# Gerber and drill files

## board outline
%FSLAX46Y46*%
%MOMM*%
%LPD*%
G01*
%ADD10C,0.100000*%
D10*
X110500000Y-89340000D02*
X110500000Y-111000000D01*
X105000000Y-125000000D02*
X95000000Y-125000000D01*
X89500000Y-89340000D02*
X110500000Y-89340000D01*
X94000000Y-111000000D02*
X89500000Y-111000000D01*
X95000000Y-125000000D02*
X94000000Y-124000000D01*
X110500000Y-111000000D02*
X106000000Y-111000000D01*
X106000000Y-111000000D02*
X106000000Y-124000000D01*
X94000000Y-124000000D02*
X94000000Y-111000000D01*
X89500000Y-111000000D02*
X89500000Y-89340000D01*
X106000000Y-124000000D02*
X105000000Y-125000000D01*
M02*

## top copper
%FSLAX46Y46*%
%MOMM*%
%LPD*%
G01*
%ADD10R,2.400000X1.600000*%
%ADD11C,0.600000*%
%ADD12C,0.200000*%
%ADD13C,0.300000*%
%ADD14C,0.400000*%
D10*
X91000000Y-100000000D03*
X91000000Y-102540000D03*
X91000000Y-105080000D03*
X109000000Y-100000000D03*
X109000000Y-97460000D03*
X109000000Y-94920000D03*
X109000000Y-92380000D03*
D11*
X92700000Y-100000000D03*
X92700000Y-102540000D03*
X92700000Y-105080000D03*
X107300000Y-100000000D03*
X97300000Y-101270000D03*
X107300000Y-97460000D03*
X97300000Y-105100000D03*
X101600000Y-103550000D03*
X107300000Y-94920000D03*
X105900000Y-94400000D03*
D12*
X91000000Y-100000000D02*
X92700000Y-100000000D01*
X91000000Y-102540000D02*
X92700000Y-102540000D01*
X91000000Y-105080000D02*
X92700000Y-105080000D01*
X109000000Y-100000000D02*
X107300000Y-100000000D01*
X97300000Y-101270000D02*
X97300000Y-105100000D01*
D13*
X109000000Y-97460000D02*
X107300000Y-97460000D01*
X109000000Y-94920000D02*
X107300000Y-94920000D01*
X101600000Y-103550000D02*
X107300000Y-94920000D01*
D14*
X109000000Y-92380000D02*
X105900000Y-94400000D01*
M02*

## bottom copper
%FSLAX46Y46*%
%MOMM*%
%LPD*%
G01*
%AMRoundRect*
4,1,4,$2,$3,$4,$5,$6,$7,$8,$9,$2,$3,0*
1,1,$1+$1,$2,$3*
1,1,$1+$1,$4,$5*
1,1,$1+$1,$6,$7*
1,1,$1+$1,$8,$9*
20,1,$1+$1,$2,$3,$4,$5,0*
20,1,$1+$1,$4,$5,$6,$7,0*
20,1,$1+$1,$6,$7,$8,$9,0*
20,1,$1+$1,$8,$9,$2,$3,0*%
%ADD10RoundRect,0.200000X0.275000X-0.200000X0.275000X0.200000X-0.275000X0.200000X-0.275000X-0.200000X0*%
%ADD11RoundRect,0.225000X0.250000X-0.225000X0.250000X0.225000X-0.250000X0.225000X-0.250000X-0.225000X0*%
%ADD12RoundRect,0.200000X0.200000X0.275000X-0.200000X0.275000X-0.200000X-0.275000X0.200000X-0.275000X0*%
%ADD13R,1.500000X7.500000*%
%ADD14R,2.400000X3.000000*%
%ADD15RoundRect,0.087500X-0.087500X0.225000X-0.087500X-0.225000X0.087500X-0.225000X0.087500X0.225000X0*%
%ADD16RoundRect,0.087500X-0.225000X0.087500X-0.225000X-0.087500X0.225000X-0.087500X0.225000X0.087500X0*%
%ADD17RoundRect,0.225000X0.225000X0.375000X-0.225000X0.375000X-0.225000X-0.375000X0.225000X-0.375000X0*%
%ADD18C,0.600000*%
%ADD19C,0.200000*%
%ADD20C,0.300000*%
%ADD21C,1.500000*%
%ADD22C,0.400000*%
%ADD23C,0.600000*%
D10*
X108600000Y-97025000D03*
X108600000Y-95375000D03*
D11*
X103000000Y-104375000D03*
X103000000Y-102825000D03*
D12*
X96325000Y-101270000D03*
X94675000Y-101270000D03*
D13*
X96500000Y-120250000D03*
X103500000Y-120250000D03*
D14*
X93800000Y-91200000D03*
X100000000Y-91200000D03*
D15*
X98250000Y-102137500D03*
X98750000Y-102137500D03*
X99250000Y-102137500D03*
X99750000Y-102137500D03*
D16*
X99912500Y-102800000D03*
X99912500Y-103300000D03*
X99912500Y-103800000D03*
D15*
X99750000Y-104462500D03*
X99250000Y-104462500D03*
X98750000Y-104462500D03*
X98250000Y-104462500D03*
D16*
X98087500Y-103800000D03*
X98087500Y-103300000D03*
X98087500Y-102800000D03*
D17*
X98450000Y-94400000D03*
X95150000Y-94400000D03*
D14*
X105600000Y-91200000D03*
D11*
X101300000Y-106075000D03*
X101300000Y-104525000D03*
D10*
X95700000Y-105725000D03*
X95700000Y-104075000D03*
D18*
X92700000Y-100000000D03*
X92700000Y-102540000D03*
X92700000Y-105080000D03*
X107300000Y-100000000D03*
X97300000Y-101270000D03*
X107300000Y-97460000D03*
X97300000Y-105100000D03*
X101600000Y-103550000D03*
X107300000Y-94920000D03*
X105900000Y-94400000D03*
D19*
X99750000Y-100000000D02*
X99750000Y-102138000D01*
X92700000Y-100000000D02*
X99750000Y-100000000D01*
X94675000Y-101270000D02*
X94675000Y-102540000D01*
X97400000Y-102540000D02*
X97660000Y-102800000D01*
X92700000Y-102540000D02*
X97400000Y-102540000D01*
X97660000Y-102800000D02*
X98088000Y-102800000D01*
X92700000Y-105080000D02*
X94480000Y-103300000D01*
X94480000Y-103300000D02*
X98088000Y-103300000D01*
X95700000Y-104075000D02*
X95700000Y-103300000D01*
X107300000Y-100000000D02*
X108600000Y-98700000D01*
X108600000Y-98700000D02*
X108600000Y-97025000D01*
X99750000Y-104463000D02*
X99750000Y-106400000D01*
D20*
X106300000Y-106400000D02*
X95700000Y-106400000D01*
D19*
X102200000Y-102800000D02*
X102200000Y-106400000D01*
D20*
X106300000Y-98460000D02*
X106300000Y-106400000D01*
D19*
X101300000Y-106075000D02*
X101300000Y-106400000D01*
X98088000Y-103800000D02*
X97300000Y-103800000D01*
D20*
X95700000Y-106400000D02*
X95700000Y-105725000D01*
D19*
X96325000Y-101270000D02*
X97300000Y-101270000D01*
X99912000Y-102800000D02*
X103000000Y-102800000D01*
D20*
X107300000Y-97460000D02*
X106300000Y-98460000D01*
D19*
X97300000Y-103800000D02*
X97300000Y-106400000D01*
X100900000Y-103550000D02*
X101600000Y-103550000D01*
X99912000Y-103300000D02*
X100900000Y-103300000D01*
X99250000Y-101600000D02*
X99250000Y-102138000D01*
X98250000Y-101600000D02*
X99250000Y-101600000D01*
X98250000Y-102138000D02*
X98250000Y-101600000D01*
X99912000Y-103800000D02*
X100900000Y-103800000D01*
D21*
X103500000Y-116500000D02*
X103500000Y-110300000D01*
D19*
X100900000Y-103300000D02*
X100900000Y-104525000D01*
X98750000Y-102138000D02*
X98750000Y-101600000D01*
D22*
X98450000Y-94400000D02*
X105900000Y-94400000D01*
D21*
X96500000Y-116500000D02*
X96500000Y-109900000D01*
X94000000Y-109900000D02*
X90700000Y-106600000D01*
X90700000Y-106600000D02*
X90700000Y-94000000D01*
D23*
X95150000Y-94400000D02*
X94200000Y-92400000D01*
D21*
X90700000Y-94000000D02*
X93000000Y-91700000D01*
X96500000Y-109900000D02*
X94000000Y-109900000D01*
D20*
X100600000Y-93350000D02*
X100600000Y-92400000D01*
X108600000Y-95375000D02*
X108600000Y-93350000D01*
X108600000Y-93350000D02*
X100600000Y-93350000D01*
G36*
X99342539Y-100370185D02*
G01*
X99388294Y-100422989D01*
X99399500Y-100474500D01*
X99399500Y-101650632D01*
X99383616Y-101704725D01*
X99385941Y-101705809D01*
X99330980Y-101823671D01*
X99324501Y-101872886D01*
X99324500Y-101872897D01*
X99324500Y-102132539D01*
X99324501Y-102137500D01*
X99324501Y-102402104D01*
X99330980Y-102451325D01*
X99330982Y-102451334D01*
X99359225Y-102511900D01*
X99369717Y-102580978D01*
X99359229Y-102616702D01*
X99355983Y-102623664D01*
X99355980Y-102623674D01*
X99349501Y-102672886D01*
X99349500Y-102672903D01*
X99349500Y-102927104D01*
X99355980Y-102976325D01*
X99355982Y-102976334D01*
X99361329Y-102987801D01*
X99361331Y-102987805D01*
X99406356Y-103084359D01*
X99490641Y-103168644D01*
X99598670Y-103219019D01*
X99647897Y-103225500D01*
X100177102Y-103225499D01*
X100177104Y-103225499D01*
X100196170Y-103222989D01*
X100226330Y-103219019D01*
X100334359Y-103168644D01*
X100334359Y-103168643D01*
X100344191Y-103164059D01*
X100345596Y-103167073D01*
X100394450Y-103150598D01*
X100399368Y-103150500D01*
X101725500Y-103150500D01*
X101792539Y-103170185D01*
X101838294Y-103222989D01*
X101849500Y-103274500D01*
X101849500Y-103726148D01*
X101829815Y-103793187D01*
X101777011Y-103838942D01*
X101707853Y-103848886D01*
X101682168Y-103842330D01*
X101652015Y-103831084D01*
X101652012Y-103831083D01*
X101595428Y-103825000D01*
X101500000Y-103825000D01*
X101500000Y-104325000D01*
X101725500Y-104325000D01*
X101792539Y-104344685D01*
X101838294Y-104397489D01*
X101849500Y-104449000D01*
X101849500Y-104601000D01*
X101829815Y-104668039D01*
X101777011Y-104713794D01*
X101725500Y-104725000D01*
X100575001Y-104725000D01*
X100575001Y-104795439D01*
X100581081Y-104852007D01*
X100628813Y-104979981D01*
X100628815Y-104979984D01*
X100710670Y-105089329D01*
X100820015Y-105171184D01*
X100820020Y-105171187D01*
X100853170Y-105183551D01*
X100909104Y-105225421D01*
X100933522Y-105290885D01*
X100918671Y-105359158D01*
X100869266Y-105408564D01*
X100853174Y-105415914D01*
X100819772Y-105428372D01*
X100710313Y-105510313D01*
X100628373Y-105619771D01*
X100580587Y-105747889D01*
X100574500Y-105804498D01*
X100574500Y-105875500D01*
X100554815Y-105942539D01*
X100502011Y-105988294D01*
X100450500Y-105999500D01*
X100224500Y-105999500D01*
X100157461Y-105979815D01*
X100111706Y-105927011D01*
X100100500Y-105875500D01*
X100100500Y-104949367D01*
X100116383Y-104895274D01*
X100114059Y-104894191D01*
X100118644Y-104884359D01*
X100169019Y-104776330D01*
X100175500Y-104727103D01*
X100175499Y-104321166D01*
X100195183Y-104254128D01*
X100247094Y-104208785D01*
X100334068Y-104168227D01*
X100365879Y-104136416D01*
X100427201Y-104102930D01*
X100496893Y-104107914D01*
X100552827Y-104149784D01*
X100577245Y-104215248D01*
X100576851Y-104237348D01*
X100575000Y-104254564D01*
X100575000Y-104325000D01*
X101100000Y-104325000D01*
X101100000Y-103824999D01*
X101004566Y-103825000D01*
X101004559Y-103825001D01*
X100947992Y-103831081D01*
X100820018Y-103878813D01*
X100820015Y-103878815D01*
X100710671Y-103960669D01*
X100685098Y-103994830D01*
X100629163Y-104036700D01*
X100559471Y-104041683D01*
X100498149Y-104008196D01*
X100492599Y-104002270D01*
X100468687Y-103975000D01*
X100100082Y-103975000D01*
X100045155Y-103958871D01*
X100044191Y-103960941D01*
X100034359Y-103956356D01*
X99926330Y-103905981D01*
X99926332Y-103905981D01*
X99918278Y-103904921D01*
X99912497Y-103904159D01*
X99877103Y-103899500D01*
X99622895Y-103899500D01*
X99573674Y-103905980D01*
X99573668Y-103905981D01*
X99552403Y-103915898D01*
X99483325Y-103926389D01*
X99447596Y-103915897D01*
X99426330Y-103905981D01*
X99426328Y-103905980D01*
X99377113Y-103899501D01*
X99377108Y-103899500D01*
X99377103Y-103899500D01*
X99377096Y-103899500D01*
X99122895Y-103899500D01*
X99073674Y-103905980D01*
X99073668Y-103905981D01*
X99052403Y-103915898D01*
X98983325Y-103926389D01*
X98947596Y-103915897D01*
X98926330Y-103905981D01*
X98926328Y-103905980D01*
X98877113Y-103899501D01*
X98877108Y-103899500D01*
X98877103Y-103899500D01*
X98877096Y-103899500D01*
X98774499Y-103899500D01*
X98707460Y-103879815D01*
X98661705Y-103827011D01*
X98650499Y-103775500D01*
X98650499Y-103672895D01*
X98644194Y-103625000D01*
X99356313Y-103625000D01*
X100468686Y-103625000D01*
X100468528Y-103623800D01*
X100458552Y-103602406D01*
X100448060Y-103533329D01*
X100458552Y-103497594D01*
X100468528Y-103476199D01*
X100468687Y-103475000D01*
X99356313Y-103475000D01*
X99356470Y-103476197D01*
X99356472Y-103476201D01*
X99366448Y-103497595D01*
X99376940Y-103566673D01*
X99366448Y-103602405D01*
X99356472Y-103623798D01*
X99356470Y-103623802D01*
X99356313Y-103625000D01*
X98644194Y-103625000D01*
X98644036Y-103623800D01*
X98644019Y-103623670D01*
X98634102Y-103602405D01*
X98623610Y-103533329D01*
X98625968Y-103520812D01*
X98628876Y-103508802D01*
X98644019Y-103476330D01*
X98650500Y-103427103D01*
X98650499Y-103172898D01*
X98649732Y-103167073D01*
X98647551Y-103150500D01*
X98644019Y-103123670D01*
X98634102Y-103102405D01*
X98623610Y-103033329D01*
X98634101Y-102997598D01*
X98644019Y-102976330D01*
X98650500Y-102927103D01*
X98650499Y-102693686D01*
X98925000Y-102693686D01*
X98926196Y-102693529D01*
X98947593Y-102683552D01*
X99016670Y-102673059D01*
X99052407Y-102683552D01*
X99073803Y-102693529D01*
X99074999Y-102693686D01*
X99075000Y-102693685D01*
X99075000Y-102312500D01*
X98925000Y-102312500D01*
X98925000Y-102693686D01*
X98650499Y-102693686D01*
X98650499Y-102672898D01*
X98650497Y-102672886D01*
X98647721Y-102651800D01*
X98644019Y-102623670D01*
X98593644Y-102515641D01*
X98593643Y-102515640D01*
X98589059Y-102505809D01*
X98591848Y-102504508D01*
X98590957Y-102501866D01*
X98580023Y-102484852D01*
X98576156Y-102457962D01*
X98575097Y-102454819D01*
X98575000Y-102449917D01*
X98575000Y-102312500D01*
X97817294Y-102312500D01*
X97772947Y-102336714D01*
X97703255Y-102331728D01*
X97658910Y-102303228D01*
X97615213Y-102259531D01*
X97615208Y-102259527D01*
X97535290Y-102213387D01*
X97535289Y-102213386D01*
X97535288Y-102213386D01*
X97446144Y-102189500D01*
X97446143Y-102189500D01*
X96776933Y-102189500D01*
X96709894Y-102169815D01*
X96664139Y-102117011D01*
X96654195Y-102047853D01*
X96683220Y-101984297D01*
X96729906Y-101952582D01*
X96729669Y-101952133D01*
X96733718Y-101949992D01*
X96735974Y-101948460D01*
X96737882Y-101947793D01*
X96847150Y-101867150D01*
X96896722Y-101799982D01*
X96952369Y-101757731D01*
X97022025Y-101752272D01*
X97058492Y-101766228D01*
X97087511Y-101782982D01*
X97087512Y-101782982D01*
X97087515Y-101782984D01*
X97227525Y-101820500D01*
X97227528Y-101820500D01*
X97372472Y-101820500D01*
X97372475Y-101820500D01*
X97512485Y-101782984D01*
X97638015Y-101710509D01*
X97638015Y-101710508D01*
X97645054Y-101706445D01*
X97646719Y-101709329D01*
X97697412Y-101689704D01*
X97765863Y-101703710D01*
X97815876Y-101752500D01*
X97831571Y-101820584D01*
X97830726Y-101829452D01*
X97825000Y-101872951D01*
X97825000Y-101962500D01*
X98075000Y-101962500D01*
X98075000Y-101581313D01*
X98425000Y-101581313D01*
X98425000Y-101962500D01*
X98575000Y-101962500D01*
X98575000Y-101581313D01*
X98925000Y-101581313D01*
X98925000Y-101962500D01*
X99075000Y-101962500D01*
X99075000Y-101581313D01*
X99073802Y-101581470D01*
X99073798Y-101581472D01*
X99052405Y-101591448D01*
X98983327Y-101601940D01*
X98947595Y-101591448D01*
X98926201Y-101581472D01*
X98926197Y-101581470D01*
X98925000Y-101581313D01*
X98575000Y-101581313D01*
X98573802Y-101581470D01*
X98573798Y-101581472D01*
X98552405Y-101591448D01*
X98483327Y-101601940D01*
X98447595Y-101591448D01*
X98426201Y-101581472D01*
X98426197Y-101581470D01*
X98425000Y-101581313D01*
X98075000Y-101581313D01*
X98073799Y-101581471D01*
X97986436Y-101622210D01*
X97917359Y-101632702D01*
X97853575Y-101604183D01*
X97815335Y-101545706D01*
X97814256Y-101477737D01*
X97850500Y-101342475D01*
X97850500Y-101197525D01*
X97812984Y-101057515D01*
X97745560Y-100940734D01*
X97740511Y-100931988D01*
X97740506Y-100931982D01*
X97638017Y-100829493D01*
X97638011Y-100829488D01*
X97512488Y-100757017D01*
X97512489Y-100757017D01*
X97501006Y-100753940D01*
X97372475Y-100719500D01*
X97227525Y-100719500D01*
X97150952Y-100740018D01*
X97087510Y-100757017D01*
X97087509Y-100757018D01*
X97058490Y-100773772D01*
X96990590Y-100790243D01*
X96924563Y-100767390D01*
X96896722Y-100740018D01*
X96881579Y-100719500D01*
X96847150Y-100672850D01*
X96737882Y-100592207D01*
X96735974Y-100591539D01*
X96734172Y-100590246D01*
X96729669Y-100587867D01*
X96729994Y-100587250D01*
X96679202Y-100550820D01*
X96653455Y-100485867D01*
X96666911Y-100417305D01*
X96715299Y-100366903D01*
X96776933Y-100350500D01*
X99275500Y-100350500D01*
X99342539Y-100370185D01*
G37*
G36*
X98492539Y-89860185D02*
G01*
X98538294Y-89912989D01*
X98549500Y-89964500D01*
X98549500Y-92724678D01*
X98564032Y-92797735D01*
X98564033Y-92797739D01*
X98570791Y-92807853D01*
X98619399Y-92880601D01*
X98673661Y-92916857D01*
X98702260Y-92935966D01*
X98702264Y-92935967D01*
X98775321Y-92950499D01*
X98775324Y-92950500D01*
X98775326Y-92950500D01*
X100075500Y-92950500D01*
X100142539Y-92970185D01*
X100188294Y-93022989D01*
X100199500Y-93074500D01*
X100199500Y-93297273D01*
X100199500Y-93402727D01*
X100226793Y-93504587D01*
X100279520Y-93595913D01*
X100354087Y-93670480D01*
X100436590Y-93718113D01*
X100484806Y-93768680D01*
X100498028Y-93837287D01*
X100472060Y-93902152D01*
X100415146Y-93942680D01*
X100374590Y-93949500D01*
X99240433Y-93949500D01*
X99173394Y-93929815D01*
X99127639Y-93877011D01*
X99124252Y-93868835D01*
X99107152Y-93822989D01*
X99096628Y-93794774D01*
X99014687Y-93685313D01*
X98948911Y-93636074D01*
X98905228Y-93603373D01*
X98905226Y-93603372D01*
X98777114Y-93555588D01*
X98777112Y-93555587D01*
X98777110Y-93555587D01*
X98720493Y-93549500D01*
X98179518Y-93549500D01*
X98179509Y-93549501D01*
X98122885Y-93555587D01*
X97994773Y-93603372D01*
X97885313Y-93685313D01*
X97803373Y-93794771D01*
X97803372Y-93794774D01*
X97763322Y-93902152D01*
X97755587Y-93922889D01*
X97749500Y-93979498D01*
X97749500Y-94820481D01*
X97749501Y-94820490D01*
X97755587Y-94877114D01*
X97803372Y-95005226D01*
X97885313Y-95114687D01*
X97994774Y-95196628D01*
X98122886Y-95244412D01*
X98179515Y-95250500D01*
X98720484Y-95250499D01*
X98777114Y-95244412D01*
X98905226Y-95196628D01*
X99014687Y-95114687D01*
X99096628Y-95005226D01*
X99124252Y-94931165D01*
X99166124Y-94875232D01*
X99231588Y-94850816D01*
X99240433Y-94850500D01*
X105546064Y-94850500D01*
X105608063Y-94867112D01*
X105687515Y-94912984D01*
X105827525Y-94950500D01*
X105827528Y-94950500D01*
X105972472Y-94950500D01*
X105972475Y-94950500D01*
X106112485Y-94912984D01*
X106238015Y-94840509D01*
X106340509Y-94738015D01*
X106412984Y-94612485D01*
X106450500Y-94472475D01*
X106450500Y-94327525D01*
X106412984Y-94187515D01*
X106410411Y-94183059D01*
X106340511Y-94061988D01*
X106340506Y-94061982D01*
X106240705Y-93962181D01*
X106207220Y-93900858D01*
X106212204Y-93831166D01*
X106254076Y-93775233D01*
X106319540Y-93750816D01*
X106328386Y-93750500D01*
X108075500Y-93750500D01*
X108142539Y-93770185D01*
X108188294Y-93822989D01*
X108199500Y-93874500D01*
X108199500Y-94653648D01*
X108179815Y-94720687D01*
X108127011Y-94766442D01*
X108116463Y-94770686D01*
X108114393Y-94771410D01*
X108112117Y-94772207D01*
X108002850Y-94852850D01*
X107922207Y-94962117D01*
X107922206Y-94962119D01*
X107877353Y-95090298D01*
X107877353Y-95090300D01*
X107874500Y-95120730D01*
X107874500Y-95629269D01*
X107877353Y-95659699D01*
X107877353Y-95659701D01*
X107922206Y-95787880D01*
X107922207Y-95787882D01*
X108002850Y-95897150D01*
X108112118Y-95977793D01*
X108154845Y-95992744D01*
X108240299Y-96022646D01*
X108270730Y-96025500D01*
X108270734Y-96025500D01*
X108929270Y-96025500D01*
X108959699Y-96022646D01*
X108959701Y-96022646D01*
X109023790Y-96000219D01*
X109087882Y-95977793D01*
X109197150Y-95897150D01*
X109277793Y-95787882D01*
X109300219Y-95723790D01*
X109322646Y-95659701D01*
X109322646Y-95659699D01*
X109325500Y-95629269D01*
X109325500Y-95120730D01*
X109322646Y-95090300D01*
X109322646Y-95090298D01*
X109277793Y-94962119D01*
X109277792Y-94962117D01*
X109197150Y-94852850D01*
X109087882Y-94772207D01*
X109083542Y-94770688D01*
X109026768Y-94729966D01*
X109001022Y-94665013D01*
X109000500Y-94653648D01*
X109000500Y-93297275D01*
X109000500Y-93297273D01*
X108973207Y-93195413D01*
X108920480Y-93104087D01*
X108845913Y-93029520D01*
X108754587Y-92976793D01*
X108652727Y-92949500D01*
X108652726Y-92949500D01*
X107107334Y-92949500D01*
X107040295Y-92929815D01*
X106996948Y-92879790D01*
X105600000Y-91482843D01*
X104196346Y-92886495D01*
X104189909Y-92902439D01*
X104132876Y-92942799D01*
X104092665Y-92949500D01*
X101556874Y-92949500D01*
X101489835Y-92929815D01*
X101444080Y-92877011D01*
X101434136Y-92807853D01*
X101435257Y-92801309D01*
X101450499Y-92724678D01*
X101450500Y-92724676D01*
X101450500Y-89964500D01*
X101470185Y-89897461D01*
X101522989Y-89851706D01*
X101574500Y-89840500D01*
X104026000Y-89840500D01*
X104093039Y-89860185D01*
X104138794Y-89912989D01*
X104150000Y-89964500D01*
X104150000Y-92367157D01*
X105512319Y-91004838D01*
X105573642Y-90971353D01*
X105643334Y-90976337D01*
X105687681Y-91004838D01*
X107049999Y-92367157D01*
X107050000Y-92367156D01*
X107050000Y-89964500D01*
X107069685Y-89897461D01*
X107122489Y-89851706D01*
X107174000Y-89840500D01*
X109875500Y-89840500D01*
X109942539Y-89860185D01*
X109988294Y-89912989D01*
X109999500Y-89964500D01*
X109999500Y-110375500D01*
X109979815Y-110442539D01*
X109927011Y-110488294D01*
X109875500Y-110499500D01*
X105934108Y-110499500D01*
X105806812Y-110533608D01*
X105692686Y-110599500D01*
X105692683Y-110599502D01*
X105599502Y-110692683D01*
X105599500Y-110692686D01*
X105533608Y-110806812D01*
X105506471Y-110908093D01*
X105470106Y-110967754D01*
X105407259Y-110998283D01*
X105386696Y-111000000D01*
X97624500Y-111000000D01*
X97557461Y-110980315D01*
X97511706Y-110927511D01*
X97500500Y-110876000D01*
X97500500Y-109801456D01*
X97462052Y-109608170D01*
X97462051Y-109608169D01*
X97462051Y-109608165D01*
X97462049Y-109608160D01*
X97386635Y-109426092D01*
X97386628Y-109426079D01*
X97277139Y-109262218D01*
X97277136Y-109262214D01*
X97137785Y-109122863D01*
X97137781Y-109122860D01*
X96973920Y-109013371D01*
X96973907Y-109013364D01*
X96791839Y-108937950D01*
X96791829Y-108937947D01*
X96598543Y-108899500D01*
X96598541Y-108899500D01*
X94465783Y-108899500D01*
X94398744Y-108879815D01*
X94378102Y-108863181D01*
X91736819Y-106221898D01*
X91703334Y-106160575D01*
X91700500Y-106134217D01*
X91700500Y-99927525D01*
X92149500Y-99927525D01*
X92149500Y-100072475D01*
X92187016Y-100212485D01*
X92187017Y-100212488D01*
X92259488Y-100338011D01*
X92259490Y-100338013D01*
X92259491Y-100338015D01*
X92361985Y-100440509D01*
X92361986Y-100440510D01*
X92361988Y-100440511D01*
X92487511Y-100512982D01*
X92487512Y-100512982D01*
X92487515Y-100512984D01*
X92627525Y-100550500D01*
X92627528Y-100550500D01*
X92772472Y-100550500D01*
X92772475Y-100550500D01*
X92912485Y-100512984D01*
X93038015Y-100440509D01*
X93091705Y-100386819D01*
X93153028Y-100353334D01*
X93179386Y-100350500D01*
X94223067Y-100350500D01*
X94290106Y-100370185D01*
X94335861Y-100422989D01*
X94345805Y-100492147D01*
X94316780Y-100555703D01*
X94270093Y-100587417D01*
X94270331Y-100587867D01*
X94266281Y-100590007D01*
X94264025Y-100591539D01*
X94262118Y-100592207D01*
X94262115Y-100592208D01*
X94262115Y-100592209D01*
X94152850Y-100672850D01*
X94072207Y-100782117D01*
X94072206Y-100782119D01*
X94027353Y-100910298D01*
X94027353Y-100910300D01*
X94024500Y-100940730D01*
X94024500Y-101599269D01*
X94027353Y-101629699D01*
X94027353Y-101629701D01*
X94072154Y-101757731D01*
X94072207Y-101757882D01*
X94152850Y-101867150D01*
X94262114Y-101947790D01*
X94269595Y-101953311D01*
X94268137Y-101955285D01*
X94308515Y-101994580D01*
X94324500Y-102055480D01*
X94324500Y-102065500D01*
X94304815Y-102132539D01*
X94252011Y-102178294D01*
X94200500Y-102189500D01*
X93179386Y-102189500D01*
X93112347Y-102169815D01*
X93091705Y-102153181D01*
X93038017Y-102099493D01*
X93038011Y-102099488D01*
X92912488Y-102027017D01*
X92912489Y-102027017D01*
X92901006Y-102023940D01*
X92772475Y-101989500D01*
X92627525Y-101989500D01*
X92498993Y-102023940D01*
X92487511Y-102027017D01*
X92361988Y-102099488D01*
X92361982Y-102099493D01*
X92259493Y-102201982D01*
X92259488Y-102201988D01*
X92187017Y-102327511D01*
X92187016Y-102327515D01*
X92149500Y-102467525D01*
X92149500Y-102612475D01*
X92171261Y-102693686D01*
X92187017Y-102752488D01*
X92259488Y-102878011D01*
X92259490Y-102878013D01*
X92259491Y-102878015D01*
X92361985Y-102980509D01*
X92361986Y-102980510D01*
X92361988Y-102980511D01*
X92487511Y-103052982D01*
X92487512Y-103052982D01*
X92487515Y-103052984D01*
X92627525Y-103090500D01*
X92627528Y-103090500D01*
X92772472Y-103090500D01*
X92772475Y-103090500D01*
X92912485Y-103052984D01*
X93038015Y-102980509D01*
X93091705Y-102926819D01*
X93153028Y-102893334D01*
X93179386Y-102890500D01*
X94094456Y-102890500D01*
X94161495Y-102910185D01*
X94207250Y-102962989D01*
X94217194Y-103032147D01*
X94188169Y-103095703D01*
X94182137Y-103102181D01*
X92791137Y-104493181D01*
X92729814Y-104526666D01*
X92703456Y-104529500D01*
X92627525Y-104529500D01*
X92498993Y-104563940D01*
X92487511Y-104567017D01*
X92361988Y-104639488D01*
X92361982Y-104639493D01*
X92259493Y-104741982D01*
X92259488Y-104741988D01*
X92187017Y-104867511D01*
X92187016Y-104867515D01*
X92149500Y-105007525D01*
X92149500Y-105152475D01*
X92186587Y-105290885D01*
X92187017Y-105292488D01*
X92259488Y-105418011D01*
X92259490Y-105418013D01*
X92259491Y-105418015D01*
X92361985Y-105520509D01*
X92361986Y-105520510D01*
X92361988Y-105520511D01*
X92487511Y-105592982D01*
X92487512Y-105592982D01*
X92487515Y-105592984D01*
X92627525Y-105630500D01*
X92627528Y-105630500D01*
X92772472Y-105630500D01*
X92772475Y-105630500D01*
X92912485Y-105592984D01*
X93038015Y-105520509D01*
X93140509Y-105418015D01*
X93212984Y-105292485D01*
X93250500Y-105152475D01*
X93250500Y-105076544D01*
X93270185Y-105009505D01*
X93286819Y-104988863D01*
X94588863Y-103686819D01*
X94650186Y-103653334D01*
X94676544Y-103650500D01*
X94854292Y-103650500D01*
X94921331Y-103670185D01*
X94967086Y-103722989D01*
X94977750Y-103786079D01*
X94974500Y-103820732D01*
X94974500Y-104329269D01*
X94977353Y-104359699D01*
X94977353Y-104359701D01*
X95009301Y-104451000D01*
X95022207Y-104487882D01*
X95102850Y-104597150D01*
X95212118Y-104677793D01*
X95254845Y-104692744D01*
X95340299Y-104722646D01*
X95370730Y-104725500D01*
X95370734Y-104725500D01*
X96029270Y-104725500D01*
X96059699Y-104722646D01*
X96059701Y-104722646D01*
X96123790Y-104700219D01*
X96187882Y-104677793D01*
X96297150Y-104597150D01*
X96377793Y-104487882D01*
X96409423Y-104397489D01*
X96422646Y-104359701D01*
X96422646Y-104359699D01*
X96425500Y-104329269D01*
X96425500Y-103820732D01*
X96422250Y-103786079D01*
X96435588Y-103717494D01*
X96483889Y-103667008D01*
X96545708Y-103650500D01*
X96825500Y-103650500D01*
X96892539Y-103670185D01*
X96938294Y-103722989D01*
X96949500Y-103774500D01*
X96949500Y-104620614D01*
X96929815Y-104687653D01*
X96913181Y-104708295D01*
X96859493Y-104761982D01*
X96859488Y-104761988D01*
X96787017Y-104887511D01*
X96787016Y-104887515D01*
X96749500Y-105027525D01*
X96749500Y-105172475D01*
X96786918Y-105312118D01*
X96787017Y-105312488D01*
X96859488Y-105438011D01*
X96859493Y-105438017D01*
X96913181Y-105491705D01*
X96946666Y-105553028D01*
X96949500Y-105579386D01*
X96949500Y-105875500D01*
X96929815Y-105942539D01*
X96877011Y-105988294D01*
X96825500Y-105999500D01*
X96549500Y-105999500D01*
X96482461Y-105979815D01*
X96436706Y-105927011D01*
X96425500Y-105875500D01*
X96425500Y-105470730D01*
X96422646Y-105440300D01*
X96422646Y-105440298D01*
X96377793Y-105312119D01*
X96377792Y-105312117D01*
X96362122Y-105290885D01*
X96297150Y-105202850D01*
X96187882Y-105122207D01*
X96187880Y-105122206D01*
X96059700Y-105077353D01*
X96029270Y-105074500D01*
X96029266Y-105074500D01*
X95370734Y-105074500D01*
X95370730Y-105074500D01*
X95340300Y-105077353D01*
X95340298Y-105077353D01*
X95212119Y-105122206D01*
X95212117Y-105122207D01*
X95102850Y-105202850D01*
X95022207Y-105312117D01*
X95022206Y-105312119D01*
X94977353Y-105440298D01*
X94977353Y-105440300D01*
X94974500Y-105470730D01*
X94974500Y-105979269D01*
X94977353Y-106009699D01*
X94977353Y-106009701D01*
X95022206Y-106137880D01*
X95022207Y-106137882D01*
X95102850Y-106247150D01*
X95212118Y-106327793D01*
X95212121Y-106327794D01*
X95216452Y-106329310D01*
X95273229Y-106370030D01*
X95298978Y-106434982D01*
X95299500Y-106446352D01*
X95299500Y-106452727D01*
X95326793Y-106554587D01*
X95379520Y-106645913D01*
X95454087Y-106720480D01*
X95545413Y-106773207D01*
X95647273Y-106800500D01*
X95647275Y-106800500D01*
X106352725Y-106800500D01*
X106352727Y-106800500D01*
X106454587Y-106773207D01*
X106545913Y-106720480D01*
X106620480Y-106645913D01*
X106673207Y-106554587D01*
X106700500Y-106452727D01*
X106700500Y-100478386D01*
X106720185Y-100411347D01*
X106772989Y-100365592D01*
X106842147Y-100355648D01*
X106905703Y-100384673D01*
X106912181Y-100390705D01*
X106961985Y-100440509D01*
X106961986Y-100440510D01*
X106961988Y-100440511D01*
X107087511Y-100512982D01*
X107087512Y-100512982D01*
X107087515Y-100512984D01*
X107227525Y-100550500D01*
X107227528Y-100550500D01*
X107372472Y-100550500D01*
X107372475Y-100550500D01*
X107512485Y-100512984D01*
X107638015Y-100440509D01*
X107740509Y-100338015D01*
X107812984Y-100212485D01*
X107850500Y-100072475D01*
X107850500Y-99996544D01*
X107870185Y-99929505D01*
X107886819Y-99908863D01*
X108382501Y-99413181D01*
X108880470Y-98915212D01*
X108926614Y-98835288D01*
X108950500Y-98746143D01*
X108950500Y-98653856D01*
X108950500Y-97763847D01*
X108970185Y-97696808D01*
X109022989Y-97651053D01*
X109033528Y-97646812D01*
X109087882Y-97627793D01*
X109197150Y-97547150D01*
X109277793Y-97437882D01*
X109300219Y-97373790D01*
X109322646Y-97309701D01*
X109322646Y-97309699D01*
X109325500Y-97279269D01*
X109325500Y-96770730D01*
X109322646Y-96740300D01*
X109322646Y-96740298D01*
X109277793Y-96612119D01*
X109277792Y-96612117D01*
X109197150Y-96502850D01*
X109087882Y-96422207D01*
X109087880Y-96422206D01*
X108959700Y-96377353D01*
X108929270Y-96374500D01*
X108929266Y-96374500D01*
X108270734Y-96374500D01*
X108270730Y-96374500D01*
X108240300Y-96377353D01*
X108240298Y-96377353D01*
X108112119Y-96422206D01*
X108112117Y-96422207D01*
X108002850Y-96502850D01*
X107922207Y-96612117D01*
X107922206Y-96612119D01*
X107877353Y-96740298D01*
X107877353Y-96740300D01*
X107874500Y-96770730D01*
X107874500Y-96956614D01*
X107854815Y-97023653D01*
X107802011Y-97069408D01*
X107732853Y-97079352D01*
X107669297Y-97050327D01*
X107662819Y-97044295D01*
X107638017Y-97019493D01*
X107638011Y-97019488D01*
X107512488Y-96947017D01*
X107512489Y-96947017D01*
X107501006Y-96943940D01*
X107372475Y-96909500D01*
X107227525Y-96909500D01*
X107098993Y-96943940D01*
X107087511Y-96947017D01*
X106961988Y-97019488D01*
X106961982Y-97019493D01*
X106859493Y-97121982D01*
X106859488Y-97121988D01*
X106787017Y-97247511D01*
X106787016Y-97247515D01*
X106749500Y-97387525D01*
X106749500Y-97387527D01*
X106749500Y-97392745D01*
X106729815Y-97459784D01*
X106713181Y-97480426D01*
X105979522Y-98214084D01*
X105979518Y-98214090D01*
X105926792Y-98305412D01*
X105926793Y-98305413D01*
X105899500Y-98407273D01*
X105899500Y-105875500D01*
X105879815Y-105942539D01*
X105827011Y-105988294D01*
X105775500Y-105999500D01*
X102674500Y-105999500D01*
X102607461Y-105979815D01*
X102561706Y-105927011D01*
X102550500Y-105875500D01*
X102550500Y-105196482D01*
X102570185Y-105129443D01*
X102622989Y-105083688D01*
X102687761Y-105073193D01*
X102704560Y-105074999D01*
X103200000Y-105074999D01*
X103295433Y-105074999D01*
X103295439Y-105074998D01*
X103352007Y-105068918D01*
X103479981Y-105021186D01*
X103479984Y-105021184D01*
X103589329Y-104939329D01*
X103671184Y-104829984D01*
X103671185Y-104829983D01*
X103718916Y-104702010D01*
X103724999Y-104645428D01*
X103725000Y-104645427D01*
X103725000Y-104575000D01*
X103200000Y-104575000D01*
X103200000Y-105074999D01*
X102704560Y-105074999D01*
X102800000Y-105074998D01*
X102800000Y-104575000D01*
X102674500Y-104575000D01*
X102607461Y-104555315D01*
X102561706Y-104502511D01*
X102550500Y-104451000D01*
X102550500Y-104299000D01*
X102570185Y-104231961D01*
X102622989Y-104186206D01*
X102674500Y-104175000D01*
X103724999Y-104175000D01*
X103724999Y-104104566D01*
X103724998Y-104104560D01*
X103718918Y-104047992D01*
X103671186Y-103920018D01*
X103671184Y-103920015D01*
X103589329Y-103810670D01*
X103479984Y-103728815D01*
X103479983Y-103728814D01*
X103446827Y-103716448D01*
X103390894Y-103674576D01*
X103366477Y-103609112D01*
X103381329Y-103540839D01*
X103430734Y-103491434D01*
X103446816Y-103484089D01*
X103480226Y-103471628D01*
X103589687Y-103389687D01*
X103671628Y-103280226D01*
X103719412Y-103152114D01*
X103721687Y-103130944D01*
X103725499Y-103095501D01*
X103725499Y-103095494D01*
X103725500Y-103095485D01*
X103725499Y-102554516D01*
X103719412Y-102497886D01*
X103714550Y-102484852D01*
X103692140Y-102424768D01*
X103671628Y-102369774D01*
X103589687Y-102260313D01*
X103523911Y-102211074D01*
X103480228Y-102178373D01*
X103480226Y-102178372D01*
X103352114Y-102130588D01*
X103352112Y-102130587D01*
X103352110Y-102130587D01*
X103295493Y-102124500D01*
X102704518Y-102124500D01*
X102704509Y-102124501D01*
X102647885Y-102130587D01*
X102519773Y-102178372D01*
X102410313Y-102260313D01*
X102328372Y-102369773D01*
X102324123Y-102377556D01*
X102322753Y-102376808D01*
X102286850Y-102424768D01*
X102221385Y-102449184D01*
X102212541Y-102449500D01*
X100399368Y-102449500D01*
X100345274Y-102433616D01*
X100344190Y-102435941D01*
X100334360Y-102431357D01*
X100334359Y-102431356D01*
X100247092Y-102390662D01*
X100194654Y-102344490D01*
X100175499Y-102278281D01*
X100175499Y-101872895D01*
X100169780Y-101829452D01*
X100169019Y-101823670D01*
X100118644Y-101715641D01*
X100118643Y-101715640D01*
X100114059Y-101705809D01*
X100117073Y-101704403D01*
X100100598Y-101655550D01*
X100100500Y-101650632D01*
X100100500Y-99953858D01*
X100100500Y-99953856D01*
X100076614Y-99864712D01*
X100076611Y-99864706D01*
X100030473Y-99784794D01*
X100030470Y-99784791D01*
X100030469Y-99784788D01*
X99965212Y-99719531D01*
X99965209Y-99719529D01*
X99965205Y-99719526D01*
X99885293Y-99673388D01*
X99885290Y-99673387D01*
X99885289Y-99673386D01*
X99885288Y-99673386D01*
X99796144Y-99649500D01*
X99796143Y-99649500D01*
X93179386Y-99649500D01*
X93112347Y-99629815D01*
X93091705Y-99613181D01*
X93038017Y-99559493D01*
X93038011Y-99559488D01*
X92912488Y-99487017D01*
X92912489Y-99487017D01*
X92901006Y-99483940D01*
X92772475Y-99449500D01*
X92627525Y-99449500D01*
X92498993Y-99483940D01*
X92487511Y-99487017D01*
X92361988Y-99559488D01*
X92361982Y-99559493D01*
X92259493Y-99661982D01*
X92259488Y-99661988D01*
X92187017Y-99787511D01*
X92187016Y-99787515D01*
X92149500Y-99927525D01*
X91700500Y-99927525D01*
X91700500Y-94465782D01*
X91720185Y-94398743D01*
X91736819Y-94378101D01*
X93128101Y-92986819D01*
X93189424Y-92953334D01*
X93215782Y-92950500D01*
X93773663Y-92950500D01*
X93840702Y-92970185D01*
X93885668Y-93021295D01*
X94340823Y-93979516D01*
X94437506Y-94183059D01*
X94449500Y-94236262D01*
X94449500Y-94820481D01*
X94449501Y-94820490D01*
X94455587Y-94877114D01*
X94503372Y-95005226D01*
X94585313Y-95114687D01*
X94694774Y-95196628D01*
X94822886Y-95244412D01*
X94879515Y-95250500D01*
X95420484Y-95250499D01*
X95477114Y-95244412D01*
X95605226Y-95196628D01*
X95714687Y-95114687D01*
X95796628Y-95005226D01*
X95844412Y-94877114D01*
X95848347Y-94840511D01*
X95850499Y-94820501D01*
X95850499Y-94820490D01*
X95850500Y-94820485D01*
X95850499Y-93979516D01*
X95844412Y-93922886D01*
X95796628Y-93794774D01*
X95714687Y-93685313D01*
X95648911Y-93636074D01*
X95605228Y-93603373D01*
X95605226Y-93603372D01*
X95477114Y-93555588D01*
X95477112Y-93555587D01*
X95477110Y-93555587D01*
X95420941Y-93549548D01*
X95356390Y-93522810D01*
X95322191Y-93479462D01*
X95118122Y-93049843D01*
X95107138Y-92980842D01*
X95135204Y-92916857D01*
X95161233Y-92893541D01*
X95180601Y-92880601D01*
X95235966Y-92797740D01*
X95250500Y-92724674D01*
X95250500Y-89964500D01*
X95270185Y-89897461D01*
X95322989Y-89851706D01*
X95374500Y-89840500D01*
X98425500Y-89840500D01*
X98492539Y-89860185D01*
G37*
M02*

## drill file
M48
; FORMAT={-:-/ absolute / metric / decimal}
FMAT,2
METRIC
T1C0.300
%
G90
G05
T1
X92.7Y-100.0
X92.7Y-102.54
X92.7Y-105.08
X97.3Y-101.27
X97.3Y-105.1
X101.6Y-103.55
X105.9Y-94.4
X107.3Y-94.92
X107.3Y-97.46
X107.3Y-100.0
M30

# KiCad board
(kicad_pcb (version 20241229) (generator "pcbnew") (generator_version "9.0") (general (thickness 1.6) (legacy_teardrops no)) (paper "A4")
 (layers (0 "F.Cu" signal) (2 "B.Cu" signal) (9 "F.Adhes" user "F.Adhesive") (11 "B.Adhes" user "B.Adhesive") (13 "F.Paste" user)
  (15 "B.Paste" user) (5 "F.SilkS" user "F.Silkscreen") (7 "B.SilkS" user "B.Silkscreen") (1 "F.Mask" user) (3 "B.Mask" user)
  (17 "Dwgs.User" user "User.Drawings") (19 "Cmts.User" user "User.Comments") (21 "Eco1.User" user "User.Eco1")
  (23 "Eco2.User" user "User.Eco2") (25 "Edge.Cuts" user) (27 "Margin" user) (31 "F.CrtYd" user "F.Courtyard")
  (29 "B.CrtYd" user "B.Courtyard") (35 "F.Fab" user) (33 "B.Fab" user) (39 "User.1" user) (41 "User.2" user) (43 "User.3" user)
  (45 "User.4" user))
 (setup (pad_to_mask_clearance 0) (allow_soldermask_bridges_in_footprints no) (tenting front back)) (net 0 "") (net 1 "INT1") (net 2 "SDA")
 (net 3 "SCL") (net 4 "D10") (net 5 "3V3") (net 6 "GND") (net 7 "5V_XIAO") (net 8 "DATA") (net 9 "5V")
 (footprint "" (layer "F.Cu") (at 100 100)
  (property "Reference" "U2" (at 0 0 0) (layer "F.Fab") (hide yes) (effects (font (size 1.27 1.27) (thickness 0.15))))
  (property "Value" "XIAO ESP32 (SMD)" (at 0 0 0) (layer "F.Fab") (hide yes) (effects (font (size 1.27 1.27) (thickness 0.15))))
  (pad "4" smd rect (at -9 0) (size 2.4 1.6) (layers "F.Cu" "F.Mask" "F.Paste") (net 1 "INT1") (thermal_bridge_angle 45))
  (pad "5" smd rect (at -9 2.54) (size 2.4 1.6) (layers "F.Cu" "F.Mask" "F.Paste") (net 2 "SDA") (thermal_bridge_angle 45))
  (pad "6" smd rect (at -9 5.08) (size 2.4 1.6) (layers "F.Cu" "F.Mask" "F.Paste") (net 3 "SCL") (thermal_bridge_angle 45))
  (pad "11" smd rect (at 9 0) (size 2.4 1.6) (layers "F.Cu" "F.Mask" "F.Paste") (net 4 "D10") (thermal_bridge_angle 45))
  (pad "12" smd rect (at 9 -2.54) (size 2.4 1.6) (layers "F.Cu" "F.Mask" "F.Paste") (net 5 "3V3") (thermal_bridge_angle 45))
  (pad "13" smd rect (at 9 -5.08) (size 2.4 1.6) (layers "F.Cu" "F.Mask" "F.Paste") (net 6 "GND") (thermal_bridge_angle 45))
  (pad "14" smd rect (at 9 -7.62) (size 2.4 1.6) (layers "F.Cu" "F.Mask" "F.Paste") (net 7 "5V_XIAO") (thermal_bridge_angle 45)))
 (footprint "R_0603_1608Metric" (layer "B.Cu") (at 108.6 96.2 90)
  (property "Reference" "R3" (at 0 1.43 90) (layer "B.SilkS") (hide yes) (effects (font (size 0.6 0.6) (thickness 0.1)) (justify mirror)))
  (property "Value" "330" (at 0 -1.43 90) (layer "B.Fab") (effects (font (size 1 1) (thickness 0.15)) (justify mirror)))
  (pad "1" smd roundrect (at -0.825 0 90) (size 0.8 0.95) (layers "B.Cu" "B.Mask" "B.Paste") (roundrect_rratio 0.25) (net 4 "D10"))
  (pad "2" smd roundrect (at 0.825 0 90) (size 0.8 0.95) (layers "B.Cu" "B.Mask" "B.Paste") (roundrect_rratio 0.25) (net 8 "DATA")))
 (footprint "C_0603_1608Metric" (layer "B.Cu") (at 103 103.6 90)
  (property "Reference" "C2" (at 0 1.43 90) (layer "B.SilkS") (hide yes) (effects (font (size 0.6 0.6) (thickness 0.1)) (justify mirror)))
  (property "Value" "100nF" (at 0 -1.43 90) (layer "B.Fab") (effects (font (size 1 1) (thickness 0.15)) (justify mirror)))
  (pad "1" smd roundrect (at -0.775 0 90) (size 0.9 0.95) (layers "B.Cu" "B.Mask" "B.Paste") (roundrect_rratio 0.25) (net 6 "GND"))
  (pad "2" smd roundrect (at 0.775 0 90) (size 0.9 0.95) (layers "B.Cu" "B.Mask" "B.Paste") (roundrect_rratio 0.25) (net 5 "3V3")))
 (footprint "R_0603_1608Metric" (layer "B.Cu") (at 95.5 101.27 180)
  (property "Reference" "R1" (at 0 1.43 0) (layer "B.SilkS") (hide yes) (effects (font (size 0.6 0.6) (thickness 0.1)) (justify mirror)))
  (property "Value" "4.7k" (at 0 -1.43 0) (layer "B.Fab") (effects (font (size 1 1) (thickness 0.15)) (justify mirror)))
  (pad "1" smd roundrect (at -0.825 0 180) (size 0.8 0.95) (layers "B.Cu" "B.Mask" "B.Paste") (roundrect_rratio 0.25) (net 5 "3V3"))
  (pad "2" smd roundrect (at 0.825 0 180) (size 0.8 0.95) (layers "B.Cu" "B.Mask" "B.Paste") (roundrect_rratio 0.25) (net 2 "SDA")))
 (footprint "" (layer "B.Cu") (at 100 120.25 180)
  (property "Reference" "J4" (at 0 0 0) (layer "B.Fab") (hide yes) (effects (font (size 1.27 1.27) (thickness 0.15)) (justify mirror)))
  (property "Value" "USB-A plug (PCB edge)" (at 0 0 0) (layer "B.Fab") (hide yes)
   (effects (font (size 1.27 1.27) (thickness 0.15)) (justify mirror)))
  (pad "1" smd rect (at 3.5 0 180) (size 1.5 7.5) (layers "B.Cu" "B.Mask") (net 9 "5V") (thermal_bridge_angle 45))
  (pad "4" smd rect (at -3.5 0 180) (size 1.5 7.5) (layers "B.Cu" "B.Mask") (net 6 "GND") (thermal_bridge_angle 45)))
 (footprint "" (layer "B.Cu") (at 93.8 91.2 180)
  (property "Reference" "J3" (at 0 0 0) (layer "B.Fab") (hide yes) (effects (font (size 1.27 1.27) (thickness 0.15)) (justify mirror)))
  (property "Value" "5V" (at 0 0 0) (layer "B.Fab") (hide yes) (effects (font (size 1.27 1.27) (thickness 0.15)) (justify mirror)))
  (pad "1" smd rect (at 0 0 180) (size 2.4 3) (layers "B.Cu" "B.Mask") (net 9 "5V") (thermal_bridge_angle 45)))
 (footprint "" (layer "B.Cu") (at 100 91.2 180)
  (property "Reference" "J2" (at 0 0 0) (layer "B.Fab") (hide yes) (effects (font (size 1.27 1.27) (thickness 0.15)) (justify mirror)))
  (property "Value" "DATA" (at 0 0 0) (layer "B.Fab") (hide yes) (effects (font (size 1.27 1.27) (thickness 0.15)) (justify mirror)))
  (pad "1" smd rect (at 0 0 180) (size 2.4 3) (layers "B.Cu" "B.Mask") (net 8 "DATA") (thermal_bridge_angle 45)))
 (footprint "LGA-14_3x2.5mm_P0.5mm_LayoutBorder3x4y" (layer "B.Cu") (at 99 103.3 -90)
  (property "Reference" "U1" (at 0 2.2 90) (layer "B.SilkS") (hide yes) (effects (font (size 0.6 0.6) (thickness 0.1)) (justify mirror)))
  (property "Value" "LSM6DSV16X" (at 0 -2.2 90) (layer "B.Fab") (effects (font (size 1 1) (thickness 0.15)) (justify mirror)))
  (pad "1" smd roundrect (at -1.1625 0.75 270) (size 0.625 0.35) (layers "B.Cu" "B.Mask" "B.Paste") (roundrect_rratio 0.25) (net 6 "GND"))
  (pad "2" smd roundrect (at -1.1625 0.25 270) (size 0.625 0.35) (layers "B.Cu" "B.Mask" "B.Paste") (roundrect_rratio 0.25) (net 6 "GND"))
  (pad "3" smd roundrect (at -1.1625 -0.25 270) (size 0.625 0.35) (layers "B.Cu" "B.Mask" "B.Paste") (roundrect_rratio 0.25) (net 6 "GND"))
  (pad "4" smd roundrect (at -1.1625 -0.75 270) (size 0.625 0.35) (layers "B.Cu" "B.Mask" "B.Paste") (roundrect_rratio 0.25) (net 1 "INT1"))
  (pad "5" smd roundrect (at -0.5 -0.9125 270) (size 0.35 0.625) (layers "B.Cu" "B.Mask" "B.Paste") (roundrect_rratio 0.25) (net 5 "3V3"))
  (pad "6" smd roundrect (at 0 -0.9125 270) (size 0.35 0.625) (layers "B.Cu" "B.Mask" "B.Paste") (roundrect_rratio 0.25) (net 6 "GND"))
  (pad "7" smd roundrect (at 0.5 -0.9125 270) (size 0.35 0.625) (layers "B.Cu" "B.Mask" "B.Paste") (roundrect_rratio 0.25) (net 6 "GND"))
  (pad "8" smd roundrect (at 1.1625 -0.75 270) (size 0.625 0.35) (layers "B.Cu" "B.Mask" "B.Paste") (roundrect_rratio 0.25) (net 5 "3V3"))
  (pad "9" smd roundrect (at 1.1625 -0.25 270) (size 0.625 0.35) (layers "B.Cu" "B.Mask" "B.Paste") (roundrect_rratio 0.25))
  (pad "10" smd roundrect (at 1.1625 0.25 270) (size 0.625 0.35) (layers "B.Cu" "B.Mask" "B.Paste") (roundrect_rratio 0.25))
  (pad "11" smd roundrect (at 1.1625 0.75 270) (size 0.625 0.35) (layers "B.Cu" "B.Mask" "B.Paste") (roundrect_rratio 0.25))
  (pad "12" smd roundrect (at 0.5 0.9125 270) (size 0.35 0.625) (layers "B.Cu" "B.Mask" "B.Paste") (roundrect_rratio 0.25) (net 5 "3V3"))
  (pad "13" smd roundrect (at 0 0.9125 270) (size 0.35 0.625) (layers "B.Cu" "B.Mask" "B.Paste") (roundrect_rratio 0.25) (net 3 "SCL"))
  (pad "14" smd roundrect (at -0.5 0.9125 270) (size 0.35 0.625) (layers "B.Cu" "B.Mask" "B.Paste") (roundrect_rratio 0.25) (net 2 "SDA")))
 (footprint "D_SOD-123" (layer "B.Cu") (at 96.8 94.4 180)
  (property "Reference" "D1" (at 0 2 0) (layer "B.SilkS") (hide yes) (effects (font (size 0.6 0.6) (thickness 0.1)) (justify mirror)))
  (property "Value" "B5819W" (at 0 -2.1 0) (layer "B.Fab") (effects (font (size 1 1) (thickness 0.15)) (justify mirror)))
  (pad "1" smd roundrect (at -1.65 0 180) (size 0.9 1.2) (layers "B.Cu" "B.Mask" "B.Paste") (roundrect_rratio 0.25) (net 7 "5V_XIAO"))
  (pad "2" smd roundrect (at 1.65 0 180) (size 0.9 1.2) (layers "B.Cu" "B.Mask" "B.Paste") (roundrect_rratio 0.25) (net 9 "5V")))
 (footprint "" (layer "B.Cu") (at 105.6 91.2 180)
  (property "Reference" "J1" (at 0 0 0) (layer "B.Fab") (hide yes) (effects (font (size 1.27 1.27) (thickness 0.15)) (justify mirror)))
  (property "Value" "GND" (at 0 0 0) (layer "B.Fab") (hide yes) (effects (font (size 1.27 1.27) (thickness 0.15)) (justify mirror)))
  (pad "1" smd rect (at 0 0 180) (size 2.4 3) (layers "B.Cu" "B.Mask") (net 6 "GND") (thermal_bridge_angle 45)))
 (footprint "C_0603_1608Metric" (layer "B.Cu") (at 101.3 105.3 90)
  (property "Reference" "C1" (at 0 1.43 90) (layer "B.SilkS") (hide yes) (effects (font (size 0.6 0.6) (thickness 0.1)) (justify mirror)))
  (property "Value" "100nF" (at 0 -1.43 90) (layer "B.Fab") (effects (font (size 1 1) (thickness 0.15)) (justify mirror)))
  (pad "1" smd roundrect (at -0.775 0 90) (size 0.9 0.95) (layers "B.Cu" "B.Mask" "B.Paste") (roundrect_rratio 0.25) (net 5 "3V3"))
  (pad "2" smd roundrect (at 0.775 0 90) (size 0.9 0.95) (layers "B.Cu" "B.Mask" "B.Paste") (roundrect_rratio 0.25) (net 6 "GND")))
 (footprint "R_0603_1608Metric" (layer "B.Cu") (at 95.7 104.9 90)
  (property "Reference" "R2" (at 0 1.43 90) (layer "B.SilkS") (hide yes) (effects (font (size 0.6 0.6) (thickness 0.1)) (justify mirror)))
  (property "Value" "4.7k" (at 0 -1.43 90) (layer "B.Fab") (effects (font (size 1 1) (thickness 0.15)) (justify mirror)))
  (pad "1" smd roundrect (at -0.825 0 90) (size 0.8 0.95) (layers "B.Cu" "B.Mask" "B.Paste") (roundrect_rratio 0.25) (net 5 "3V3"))
  (pad "2" smd roundrect (at 0.825 0 90) (size 0.8 0.95) (layers "B.Cu" "B.Mask" "B.Paste") (roundrect_rratio 0.25) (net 3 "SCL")))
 (gr_line (start 110.5 89.34) (end 110.5 111) (stroke (width 0.1) (type default)) (layer "Edge.Cuts"))
 (gr_line (start 105 125) (end 95 125) (stroke (width 0.1) (type default)) (layer "Edge.Cuts"))
 (gr_line (start 89.5 89.34) (end 110.5 89.34) (stroke (width 0.1) (type default)) (layer "Edge.Cuts"))
 (gr_line (start 94 111) (end 89.5 111) (stroke (width 0.1) (type default)) (layer "Edge.Cuts"))
 (gr_line (start 95 125) (end 94 124) (stroke (width 0.1) (type default)) (layer "Edge.Cuts"))
 (gr_line (start 110.5 111) (end 106 111) (stroke (width 0.1) (type default)) (layer "Edge.Cuts"))
 (gr_line (start 106 111) (end 106 124) (stroke (width 0.1) (type default)) (layer "Edge.Cuts"))
 (gr_line (start 94 124) (end 94 111) (stroke (width 0.1) (type default)) (layer "Edge.Cuts"))
 (gr_line (start 89.5 111) (end 89.5 89.34) (stroke (width 0.1) (type default)) (layer "Edge.Cuts"))
 (gr_line (start 106 124) (end 105 125) (stroke (width 0.1) (type default)) (layer "Edge.Cuts"))
 (segment (start 91 100) (end 92.7 100) (width 0.2) (layer "F.Cu") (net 1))
 (via (at 92.7 100) (size 0.6) (drill 0.3) (layers "F.Cu" "B.Cu") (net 1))
 (segment (start 99.75 100) (end 99.75 102.138) (width 0.2) (layer "B.Cu") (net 1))
 (segment (start 92.7 100) (end 99.75 100) (width 0.2) (layer "B.Cu") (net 1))
 (segment (start 91 102.54) (end 92.7 102.54) (width 0.2) (layer "F.Cu") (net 2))
 (via (at 92.7 102.54) (size 0.6) (drill 0.3) (layers "F.Cu" "B.Cu") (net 2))
 (segment (start 94.675 101.27) (end 94.675 102.54) (width 0.2) (layer "B.Cu") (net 2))
 (segment (start 97.4 102.54) (end 97.66 102.8) (width 0.2) (layer "B.Cu") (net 2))
 (segment (start 92.7 102.54) (end 97.4 102.54) (width 0.2) (layer "B.Cu") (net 2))
 (segment (start 97.66 102.8) (end 98.088 102.8) (width 0.2) (layer "B.Cu") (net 2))
 (segment (start 91 105.08) (end 92.7 105.08) (width 0.2) (layer "F.Cu") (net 3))
 (via (at 92.7 105.08) (size 0.6) (drill 0.3) (layers "F.Cu" "B.Cu") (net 3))
 (segment (start 92.7 105.08) (end 94.48 103.3) (width 0.2) (layer "B.Cu") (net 3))
 (segment (start 94.48 103.3) (end 98.088 103.3) (width 0.2) (layer "B.Cu") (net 3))
 (segment (start 95.7 104.075) (end 95.7 103.3) (width 0.2) (layer "B.Cu") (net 3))
 (segment (start 109 100) (end 107.3 100) (width 0.2) (layer "F.Cu") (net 4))
 (via (at 107.3 100) (size 0.6) (drill 0.3) (layers "F.Cu" "B.Cu") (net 4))
 (segment (start 107.3 100) (end 108.6 98.7) (width 0.2) (layer "B.Cu") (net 4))
 (segment (start 108.6 98.7) (end 108.6 97.025) (width 0.2) (layer "B.Cu") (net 4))
 (segment (start 97.3 101.27) (end 97.3 105.1) (width 0.2) (layer "F.Cu") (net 5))
 (segment (start 109 97.46) (end 107.3 97.46) (width 0.3) (layer "F.Cu") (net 5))
 (via (at 97.3 101.27) (size 0.6) (drill 0.3) (layers "F.Cu" "B.Cu") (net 5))
 (via (at 107.3 97.46) (size 0.6) (drill 0.3) (layers "F.Cu" "B.Cu") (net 5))
 (via (at 97.3 105.1) (size 0.6) (drill 0.3) (layers "F.Cu" "B.Cu") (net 5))
 (segment (start 99.75 104.463) (end 99.75 106.4) (width 0.2) (layer "B.Cu") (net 5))
 (segment (start 106.3 106.4) (end 95.7 106.4) (width 0.3) (layer "B.Cu") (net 5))
 (segment (start 102.2 102.8) (end 102.2 106.4) (width 0.2) (layer "B.Cu") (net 5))
 (segment (start 106.3 98.46) (end 106.3 106.4) (width 0.3) (layer "B.Cu") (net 5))
 (segment (start 101.3 106.075) (end 101.3 106.4) (width 0.2) (layer "B.Cu") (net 5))
 (segment (start 98.088 103.8) (end 97.3 103.8) (width 0.2) (layer "B.Cu") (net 5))
 (segment (start 95.7 106.4) (end 95.7 105.725) (width 0.3) (layer "B.Cu") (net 5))
 (segment (start 96.325 101.27) (end 97.3 101.27) (width 0.2) (layer "B.Cu") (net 5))
 (segment (start 99.912 102.8) (end 103 102.8) (width 0.2) (layer "B.Cu") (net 5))
 (segment (start 107.3 97.46) (end 106.3 98.46) (width 0.3) (layer "B.Cu") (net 5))
 (segment (start 97.3 103.8) (end 97.3 106.4) (width 0.2) (layer "B.Cu") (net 5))
 (segment (start 109 94.92) (end 107.3 94.92) (width 0.3) (layer "F.Cu") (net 6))
 (segment (start 101.6 103.55) (end 107.3 94.92) (width 0.3) (layer "F.Cu") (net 6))
 (via (at 101.6 103.55) (size 0.6) (drill 0.3) (layers "F.Cu" "B.Cu") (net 6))
 (via (at 107.3 94.92) (size 0.6) (drill 0.3) (layers "F.Cu" "B.Cu") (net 6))
 (segment (start 100.9 103.55) (end 101.6 103.55) (width 0.2) (layer "B.Cu") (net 6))
 (segment (start 99.912 103.3) (end 100.9 103.3) (width 0.2) (layer "B.Cu") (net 6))
 (segment (start 99.25 101.6) (end 99.25 102.138) (width 0.2) (layer "B.Cu") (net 6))
 (segment (start 98.25 101.6) (end 99.25 101.6) (width 0.2) (layer "B.Cu") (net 6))
 (segment (start 98.25 102.138) (end 98.25 101.6) (width 0.2) (layer "B.Cu") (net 6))
 (segment (start 99.912 103.8) (end 100.9 103.8) (width 0.2) (layer "B.Cu") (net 6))
 (segment (start 103.5 116.5) (end 103.5 110.3) (width 1.5) (layer "B.Cu") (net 6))
 (segment (start 100.9 103.3) (end 100.9 104.525) (width 0.2) (layer "B.Cu") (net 6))
 (segment (start 98.75 102.138) (end 98.75 101.6) (width 0.2) (layer "B.Cu") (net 6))
 (segment (start 109 92.38) (end 105.9 94.4) (width 0.4) (layer "F.Cu") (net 7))
 (via (at 105.9 94.4) (size 0.6) (drill 0.3) (layers "F.Cu" "B.Cu") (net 7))
 (segment (start 98.45 94.4) (end 105.9 94.4) (width 0.4) (layer "B.Cu") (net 7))
 (segment (start 96.5 116.5) (end 96.5 109.9) (width 1.5) (layer "B.Cu") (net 9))
 (segment (start 94 109.9) (end 90.7 106.6) (width 1.5) (layer "B.Cu") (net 9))
 (segment (start 90.7 106.6) (end 90.7 94) (width 1.5) (layer "B.Cu") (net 9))
 (segment (start 95.15 94.4) (end 94.2 92.4) (width 0.6) (layer "B.Cu") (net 9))
 (segment (start 90.7 94) (end 93 91.7) (width 1.5) (layer "B.Cu") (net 9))
 (segment (start 96.5 109.9) (end 94 109.9) (width 1.5) (layer "B.Cu") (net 9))
 (segment (start 100.6 93.35) (end 100.6 92.4) (width 0.3) (layer "B.Cu") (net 8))
 (segment (start 108.6 95.375) (end 108.6 93.35) (width 0.3) (layer "B.Cu") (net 8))
 (segment (start 108.6 93.35) (end 100.6 93.35) (width 0.3) (layer "B.Cu") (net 8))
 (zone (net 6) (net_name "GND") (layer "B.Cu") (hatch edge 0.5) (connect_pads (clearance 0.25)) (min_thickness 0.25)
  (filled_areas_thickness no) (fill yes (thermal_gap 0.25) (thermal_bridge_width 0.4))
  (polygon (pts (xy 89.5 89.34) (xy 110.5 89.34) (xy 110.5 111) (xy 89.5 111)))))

